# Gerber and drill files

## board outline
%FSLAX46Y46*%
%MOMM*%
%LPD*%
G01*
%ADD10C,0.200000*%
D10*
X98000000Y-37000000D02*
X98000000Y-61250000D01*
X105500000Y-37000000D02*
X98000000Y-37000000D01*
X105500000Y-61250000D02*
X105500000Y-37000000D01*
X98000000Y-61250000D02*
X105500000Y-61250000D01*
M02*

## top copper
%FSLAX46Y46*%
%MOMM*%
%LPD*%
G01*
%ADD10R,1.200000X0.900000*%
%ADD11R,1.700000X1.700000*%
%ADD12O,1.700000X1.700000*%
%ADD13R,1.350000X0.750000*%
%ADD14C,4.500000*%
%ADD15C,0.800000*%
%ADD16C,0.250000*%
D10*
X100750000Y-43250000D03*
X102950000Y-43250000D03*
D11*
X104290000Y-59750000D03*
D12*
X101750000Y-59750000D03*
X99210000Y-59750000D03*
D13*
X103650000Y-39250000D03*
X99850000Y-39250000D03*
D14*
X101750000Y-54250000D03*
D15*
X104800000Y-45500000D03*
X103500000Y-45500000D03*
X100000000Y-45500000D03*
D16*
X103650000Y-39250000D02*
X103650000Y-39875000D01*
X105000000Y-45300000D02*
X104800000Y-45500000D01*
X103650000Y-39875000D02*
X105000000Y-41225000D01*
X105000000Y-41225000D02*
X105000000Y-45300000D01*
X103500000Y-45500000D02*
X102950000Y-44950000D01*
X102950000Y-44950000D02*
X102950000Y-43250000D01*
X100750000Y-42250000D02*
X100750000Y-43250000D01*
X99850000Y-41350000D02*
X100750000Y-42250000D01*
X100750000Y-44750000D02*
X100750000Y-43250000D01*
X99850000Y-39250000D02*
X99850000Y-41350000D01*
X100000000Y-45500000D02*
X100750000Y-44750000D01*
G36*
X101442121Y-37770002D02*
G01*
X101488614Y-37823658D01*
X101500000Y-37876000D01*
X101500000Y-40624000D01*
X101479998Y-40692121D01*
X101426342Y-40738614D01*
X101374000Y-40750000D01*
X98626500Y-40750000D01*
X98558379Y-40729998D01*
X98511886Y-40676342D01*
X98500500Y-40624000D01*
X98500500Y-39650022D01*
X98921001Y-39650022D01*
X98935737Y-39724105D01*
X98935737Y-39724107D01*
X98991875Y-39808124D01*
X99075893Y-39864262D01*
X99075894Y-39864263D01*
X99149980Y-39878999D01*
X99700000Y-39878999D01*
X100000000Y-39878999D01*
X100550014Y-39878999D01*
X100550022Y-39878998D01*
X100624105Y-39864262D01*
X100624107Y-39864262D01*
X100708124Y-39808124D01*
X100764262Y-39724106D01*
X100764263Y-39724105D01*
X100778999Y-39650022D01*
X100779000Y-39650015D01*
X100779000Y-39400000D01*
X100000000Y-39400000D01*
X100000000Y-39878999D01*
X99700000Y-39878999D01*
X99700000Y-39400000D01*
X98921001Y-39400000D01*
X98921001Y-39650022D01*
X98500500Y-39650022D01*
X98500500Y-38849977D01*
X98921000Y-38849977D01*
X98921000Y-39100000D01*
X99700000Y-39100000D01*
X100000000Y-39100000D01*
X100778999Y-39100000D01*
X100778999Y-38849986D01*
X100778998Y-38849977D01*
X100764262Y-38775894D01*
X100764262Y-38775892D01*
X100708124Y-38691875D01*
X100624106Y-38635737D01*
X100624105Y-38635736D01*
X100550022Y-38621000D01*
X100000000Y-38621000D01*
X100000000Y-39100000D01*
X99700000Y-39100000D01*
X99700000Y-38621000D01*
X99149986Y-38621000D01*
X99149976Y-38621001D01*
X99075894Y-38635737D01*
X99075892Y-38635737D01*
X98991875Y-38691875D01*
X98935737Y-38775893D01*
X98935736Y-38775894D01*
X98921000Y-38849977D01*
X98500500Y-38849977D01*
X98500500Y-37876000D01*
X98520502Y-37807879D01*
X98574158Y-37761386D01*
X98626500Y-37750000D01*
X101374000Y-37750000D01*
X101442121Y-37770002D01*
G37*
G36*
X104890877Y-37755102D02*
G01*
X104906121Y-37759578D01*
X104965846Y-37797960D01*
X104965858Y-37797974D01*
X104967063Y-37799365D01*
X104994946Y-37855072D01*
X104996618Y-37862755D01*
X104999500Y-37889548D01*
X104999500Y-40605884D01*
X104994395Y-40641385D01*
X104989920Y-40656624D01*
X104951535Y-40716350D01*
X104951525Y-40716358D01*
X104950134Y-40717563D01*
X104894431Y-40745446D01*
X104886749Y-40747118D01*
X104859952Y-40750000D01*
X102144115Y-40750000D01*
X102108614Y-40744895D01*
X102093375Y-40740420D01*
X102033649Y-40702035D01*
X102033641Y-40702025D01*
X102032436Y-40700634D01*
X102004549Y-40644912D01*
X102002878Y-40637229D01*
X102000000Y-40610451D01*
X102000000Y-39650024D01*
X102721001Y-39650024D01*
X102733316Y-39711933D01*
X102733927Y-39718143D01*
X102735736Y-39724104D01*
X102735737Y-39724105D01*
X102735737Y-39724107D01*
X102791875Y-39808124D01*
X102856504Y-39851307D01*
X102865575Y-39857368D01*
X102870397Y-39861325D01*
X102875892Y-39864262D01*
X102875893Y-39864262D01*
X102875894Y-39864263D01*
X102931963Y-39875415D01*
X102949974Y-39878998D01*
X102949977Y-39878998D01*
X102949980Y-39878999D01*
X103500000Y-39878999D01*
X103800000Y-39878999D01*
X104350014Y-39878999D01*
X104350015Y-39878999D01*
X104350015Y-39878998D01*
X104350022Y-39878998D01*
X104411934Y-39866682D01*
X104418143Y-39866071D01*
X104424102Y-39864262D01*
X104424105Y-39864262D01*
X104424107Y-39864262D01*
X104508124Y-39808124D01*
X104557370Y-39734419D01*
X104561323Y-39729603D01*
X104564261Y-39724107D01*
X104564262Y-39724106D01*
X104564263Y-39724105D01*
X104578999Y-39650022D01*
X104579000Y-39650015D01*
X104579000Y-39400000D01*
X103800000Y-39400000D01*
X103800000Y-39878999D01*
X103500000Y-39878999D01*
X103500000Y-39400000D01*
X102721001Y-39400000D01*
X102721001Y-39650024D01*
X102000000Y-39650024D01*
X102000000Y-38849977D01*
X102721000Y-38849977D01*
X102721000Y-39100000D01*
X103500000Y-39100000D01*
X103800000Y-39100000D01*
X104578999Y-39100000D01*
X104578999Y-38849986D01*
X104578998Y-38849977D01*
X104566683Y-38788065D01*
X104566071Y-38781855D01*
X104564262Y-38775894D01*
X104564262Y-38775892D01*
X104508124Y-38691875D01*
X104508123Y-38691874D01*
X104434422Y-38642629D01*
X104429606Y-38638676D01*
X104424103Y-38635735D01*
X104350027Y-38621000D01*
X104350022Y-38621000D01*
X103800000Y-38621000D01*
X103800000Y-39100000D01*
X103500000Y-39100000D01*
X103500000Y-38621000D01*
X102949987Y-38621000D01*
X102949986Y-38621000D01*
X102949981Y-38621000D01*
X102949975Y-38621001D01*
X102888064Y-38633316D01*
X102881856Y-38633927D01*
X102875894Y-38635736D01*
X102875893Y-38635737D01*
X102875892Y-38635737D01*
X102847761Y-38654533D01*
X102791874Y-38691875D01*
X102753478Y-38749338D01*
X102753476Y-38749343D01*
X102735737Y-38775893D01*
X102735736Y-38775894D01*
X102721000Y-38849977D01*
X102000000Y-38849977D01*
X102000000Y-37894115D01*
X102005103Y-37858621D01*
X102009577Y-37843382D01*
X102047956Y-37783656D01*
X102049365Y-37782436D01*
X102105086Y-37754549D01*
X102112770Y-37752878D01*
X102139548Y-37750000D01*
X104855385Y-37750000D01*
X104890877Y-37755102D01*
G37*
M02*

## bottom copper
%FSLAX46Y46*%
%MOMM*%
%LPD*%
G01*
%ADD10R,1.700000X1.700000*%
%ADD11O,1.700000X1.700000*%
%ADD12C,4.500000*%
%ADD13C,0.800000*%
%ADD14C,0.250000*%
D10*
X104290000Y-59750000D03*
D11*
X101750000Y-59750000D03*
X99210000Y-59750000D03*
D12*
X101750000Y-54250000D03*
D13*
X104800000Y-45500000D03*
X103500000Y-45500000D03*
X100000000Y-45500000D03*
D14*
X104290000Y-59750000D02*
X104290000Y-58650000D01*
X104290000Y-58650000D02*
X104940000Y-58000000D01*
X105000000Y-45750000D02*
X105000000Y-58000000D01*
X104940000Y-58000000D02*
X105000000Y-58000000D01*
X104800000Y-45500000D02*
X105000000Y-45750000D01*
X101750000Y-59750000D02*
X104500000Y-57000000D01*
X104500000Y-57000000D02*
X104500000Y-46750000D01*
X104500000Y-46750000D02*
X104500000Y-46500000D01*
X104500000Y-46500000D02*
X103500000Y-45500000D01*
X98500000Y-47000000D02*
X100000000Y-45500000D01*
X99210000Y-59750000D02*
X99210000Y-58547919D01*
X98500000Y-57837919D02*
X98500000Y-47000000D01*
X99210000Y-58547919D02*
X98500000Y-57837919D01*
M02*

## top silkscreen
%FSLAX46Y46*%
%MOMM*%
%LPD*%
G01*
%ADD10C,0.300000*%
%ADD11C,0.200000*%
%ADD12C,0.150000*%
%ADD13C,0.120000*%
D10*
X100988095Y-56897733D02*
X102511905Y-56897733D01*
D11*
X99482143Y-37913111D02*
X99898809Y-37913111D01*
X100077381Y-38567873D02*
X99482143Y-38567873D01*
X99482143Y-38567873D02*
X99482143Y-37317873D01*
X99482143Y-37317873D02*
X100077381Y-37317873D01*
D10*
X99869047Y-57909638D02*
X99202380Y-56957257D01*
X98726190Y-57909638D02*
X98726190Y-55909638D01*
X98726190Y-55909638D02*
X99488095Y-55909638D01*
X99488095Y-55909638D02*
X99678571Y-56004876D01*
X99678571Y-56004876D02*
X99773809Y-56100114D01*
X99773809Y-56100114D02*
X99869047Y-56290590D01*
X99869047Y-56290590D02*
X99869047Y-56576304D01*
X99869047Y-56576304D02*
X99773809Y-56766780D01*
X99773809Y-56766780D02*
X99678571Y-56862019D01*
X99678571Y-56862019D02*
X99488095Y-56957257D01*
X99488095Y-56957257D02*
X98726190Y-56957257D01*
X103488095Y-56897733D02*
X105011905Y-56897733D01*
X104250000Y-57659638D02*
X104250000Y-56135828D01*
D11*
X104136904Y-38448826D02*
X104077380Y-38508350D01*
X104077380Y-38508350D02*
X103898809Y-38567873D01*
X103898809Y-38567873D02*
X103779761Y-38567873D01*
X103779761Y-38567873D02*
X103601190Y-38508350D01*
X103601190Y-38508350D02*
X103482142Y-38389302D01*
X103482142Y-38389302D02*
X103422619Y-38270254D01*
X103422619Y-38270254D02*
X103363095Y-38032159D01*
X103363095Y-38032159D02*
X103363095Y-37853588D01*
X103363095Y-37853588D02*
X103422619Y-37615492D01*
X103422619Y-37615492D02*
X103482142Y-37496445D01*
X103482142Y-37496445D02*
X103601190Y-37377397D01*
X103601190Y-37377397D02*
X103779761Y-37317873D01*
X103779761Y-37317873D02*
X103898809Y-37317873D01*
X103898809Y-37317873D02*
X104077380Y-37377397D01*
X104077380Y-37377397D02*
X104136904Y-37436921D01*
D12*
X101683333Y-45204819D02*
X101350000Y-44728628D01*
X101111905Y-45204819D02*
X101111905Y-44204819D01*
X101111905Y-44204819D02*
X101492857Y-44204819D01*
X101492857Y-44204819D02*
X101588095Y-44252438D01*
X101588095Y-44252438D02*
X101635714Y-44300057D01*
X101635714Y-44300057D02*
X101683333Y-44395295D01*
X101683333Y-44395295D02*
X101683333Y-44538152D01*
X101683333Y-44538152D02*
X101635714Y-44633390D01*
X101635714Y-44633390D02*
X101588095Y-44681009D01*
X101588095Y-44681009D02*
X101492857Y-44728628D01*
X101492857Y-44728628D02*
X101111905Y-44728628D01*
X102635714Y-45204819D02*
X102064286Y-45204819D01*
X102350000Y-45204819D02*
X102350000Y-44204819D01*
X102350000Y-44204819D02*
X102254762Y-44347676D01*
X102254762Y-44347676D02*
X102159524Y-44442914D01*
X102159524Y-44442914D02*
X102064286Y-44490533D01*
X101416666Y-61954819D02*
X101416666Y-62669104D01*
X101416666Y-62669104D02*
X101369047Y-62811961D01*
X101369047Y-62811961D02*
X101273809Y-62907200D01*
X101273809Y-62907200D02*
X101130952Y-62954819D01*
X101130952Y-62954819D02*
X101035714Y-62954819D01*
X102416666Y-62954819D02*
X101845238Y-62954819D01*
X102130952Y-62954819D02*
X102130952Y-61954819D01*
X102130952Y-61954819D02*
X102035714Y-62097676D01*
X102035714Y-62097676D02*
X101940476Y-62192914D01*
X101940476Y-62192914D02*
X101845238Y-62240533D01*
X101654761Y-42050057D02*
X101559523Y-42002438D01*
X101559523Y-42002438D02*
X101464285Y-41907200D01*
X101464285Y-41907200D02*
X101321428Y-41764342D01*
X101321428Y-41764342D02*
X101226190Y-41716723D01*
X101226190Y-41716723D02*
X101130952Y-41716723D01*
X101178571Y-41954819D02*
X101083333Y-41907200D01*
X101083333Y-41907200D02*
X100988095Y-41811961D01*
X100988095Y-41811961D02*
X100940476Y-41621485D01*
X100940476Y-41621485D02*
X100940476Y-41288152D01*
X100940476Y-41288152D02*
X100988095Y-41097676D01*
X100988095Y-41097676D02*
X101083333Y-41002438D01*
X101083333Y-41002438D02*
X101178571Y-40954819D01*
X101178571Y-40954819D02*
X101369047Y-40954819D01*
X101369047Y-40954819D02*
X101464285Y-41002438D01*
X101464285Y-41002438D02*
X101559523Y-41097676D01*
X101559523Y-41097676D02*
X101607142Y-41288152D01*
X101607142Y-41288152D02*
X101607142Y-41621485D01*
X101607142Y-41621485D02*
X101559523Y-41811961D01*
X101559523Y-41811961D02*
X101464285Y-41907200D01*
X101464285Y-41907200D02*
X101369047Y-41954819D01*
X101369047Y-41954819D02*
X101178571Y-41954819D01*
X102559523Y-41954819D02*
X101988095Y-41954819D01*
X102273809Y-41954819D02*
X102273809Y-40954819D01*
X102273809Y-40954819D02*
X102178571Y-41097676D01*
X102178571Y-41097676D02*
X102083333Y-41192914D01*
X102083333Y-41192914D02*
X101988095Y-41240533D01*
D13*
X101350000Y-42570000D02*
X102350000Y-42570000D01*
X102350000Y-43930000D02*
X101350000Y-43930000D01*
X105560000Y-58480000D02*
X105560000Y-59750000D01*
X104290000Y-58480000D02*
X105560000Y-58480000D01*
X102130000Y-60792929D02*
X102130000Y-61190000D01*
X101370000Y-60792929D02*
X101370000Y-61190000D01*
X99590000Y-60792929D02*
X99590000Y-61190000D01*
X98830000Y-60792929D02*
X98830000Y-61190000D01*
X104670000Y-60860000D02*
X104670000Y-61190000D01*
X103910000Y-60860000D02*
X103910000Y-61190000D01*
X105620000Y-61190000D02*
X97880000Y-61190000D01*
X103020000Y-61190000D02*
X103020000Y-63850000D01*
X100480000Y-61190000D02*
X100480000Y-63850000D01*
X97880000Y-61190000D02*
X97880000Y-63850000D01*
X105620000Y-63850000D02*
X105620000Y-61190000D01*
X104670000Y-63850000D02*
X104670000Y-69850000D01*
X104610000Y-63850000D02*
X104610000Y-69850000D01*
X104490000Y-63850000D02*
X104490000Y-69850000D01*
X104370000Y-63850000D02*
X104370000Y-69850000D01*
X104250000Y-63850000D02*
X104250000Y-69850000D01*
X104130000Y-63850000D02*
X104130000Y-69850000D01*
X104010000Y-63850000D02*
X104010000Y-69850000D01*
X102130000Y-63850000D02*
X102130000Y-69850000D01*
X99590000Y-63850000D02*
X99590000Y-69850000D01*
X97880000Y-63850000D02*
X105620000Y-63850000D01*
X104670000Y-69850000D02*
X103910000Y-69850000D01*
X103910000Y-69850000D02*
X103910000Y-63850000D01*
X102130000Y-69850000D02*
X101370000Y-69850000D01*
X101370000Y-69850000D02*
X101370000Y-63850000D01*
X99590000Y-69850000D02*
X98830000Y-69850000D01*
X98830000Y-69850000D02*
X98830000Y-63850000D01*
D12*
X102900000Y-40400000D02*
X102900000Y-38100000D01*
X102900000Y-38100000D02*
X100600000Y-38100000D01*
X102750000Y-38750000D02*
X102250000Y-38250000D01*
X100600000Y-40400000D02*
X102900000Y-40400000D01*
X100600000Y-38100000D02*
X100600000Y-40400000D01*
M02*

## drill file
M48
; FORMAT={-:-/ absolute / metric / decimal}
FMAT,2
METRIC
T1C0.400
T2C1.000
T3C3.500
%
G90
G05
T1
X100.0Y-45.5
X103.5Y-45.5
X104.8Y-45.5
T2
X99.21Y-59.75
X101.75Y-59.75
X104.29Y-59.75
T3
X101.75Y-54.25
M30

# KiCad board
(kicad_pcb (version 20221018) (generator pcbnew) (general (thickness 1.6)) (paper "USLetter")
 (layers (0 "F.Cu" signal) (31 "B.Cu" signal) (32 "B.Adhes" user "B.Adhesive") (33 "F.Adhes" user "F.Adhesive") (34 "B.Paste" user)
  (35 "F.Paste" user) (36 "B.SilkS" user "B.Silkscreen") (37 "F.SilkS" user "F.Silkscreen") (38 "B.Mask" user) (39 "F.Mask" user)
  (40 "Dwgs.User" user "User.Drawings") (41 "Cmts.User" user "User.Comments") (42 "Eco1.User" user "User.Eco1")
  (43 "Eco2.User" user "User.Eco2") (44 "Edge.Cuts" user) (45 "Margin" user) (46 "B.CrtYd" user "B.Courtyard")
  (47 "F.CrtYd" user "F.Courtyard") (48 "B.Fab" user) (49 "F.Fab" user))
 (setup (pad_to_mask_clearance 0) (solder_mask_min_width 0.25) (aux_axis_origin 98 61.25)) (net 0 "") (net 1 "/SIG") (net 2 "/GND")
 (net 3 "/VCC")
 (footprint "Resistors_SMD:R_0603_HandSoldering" (layer "F.Cu") (at 101.85 43.25)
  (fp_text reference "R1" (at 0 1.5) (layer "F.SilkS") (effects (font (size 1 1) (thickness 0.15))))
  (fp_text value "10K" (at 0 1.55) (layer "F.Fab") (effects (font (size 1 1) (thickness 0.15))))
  (fp_line (start -0.5 -0.68) (end 0.5 -0.68) (stroke (width 0.12) (type solid)) (layer "F.SilkS"))
  (fp_line (start 0.5 0.68) (end -0.5 0.68) (stroke (width 0.12) (type solid)) (layer "F.SilkS"))
  (pad "1" smd rect (at -1.1 0) (size 1.2 0.9) (layers "F.Cu" "F.Paste" "F.Mask") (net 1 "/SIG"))
  (pad "2" smd rect (at 1.1 0) (size 1.2 0.9) (layers "F.Cu" "F.Paste" "F.Mask") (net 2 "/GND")))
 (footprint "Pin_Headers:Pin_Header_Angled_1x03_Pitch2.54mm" (layer "F.Cu") (at 104.29 59.75 -90)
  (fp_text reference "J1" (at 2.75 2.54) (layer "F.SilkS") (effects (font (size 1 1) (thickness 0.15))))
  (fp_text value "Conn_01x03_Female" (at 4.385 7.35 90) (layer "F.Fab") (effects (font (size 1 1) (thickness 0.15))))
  (fp_line (start -1.27 -1.27) (end 0 -1.27) (stroke (width 0.12) (type solid)) (layer "F.SilkS"))
  (fp_line (start -1.27 0) (end -1.27 -1.27) (stroke (width 0.12) (type solid)) (layer "F.SilkS"))
  (fp_line (start 1.042929 2.16) (end 1.44 2.16) (stroke (width 0.12) (type solid)) (layer "F.SilkS"))
  (fp_line (start 1.042929 2.92) (end 1.44 2.92) (stroke (width 0.12) (type solid)) (layer "F.SilkS"))
  (fp_line (start 1.042929 4.7) (end 1.44 4.7) (stroke (width 0.12) (type solid)) (layer "F.SilkS"))
  (fp_line (start 1.042929 5.46) (end 1.44 5.46) (stroke (width 0.12) (type solid)) (layer "F.SilkS"))
  (fp_line (start 1.11 -0.38) (end 1.44 -0.38) (stroke (width 0.12) (type solid)) (layer "F.SilkS"))
  (fp_line (start 1.11 0.38) (end 1.44 0.38) (stroke (width 0.12) (type solid)) (layer "F.SilkS"))
  (fp_line (start 1.44 -1.33) (end 1.44 6.41) (stroke (width 0.12) (type solid)) (layer "F.SilkS"))
  (fp_line (start 1.44 1.27) (end 4.1 1.27) (stroke (width 0.12) (type solid)) (layer "F.SilkS"))
  (fp_line (start 1.44 3.81) (end 4.1 3.81) (stroke (width 0.12) (type solid)) (layer "F.SilkS"))
  (fp_line (start 1.44 6.41) (end 4.1 6.41) (stroke (width 0.12) (type solid)) (layer "F.SilkS"))
  (fp_line (start 4.1 -1.33) (end 1.44 -1.33) (stroke (width 0.12) (type solid)) (layer "F.SilkS"))
  (fp_line (start 4.1 -0.38) (end 10.1 -0.38) (stroke (width 0.12) (type solid)) (layer "F.SilkS"))
  (fp_line (start 4.1 -0.32) (end 10.1 -0.32) (stroke (width 0.12) (type solid)) (layer "F.SilkS"))
  (fp_line (start 4.1 -0.2) (end 10.1 -0.2) (stroke (width 0.12) (type solid)) (layer "F.SilkS"))
  (fp_line (start 4.1 -0.08) (end 10.1 -0.08) (stroke (width 0.12) (type solid)) (layer "F.SilkS"))
  (fp_line (start 4.1 0.04) (end 10.1 0.04) (stroke (width 0.12) (type solid)) (layer "F.SilkS"))
  (fp_line (start 4.1 0.16) (end 10.1 0.16) (stroke (width 0.12) (type solid)) (layer "F.SilkS"))
  (fp_line (start 4.1 0.28) (end 10.1 0.28) (stroke (width 0.12) (type solid)) (layer "F.SilkS"))
  (fp_line (start 4.1 2.16) (end 10.1 2.16) (stroke (width 0.12) (type solid)) (layer "F.SilkS"))
  (fp_line (start 4.1 4.7) (end 10.1 4.7) (stroke (width 0.12) (type solid)) (layer "F.SilkS"))
  (fp_line (start 4.1 6.41) (end 4.1 -1.33) (stroke (width 0.12) (type solid)) (layer "F.SilkS"))
  (fp_line (start 10.1 -0.38) (end 10.1 0.38) (stroke (width 0.12) (type solid)) (layer "F.SilkS"))
  (fp_line (start 10.1 0.38) (end 4.1 0.38) (stroke (width 0.12) (type solid)) (layer "F.SilkS"))
  (fp_line (start 10.1 2.16) (end 10.1 2.92) (stroke (width 0.12) (type solid)) (layer "F.SilkS"))
  (fp_line (start 10.1 2.92) (end 4.1 2.92) (stroke (width 0.12) (type solid)) (layer "F.SilkS"))
  (fp_line (start 10.1 4.7) (end 10.1 5.46) (stroke (width 0.12) (type solid)) (layer "F.SilkS"))
  (fp_line (start 10.1 5.46) (end 4.1 5.46) (stroke (width 0.12) (type solid)) (layer "F.SilkS"))
  (pad "1" thru_hole rect (at 0 0 270) (size 1.7 1.7) (drill 1) (layers "*.Cu" "*.Mask") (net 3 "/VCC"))
  (pad "2" thru_hole oval (at 0 2.54 270) (size 1.7 1.7) (drill 1) (layers "*.Cu" "*.Mask") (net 2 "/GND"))
  (pad "3" thru_hole oval (at 0 5.08 270) (size 1.7 1.7) (drill 1) (layers "*.Cu" "*.Mask") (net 1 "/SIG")))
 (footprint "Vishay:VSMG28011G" (layer "F.Cu") (at 101.75 39.25 180)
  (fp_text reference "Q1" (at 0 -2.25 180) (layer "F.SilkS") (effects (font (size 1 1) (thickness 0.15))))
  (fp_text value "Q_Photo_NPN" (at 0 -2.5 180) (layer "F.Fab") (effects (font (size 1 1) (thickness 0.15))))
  (fp_line (start -1.15 -1.15) (end -1.15 1.15) (stroke (width 0.15) (type solid)) (layer "F.SilkS"))
  (fp_line (start -1.15 1.15) (end 1.15 1.15) (stroke (width 0.15) (type solid)) (layer "F.SilkS"))
  (fp_line (start -1 0.5) (end -0.5 1) (stroke (width 0.15) (type solid)) (layer "F.SilkS"))
  (fp_line (start 1.15 -1.15) (end -1.15 -1.15) (stroke (width 0.15) (type solid)) (layer "F.SilkS"))
  (fp_line (start 1.15 1.15) (end 1.15 -1.15) (stroke (width 0.15) (type solid)) (layer "F.SilkS"))
  (pad "1" smd rect (at -1.9 0 180) (size 1.35 0.75) (layers "F.Cu" "F.Paste" "F.Mask") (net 3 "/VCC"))
  (pad "2" smd rect (at 1.9 0 180) (size 1.35 0.75) (layers "F.Cu" "F.Paste" "F.Mask") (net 1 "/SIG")))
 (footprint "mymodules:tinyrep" (layer "B.Cu") (at 101.75 44.5 90)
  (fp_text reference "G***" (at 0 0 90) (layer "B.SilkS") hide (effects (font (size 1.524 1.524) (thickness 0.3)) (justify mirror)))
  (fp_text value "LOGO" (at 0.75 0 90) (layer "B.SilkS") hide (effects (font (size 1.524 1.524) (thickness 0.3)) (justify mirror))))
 (gr_line (start 98 37) (end 98 61.25) (stroke (width 0.2) (type solid)) (layer "Edge.Cuts"))
 (gr_line (start 105.5 37) (end 98 37) (stroke (width 0.2) (type solid)) (layer "Edge.Cuts"))
 (gr_line (start 105.5 61.25) (end 105.5 37) (stroke (width 0.2) (type solid)) (layer "Edge.Cuts"))
 (gr_line (start 98 61.25) (end 105.5 61.25) (stroke (width 0.2) (type solid)) (layer "Edge.Cuts"))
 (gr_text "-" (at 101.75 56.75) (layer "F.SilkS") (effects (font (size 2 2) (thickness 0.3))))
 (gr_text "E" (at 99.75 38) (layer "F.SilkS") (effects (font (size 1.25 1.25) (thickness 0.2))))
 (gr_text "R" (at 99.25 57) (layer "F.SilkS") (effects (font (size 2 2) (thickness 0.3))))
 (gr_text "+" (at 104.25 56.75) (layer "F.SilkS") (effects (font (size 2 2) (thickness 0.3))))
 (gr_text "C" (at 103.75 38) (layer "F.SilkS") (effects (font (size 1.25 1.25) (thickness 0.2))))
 (via (at 101.75 54.25) (size 4.5) (drill 3.5) (layers "F.Cu" "B.Cu") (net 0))
 (segment (start 103.65 39.25) (end 103.65 39.875) (width 0.25) (layer "F.Cu") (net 3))
 (segment (start 105 45.3) (end 104.8 45.5) (width 0.25) (layer "F.Cu") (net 3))
 (segment (start 103.65 39.875) (end 105 41.225) (width 0.25) (layer "F.Cu") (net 3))
 (segment (start 105 41.225) (end 105 45.3) (width 0.25) (layer "F.Cu") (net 3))
 (via (at 104.8 45.5) (size 0.8) (drill 0.4) (layers "F.Cu" "B.Cu") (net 3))
 (segment (start 104.29 59.75) (end 104.29 58.65) (width 0.25) (layer "B.Cu") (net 3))
 (segment (start 104.29 58.65) (end 104.94 58) (width 0.25) (layer "B.Cu") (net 3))
 (segment (start 105 45.75) (end 105 58) (width 0.25) (layer "B.Cu") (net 3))
 (segment (start 104.94 58) (end 105 58) (width 0.25) (layer "B.Cu") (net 3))
 (segment (start 104.8 45.5) (end 105 45.75) (width 0.25) (layer "B.Cu") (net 3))
 (segment (start 103.5 45.5) (end 102.95 44.95) (width 0.25) (layer "F.Cu") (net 2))
 (segment (start 102.95 44.95) (end 102.95 43.25) (width 0.25) (layer "F.Cu") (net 2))
 (via (at 103.5 45.5) (size 0.8) (drill 0.4) (layers "F.Cu" "B.Cu") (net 2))
 (segment (start 101.75 59.75) (end 104.5 57) (width 0.25) (layer "B.Cu") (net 2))
 (segment (start 104.5 57) (end 104.5 46.75) (width 0.25) (layer "B.Cu") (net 2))
 (segment (start 104.5 46.75) (end 104.5 46.5) (width 0.25) (layer "B.Cu") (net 2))
 (segment (start 104.5 46.5) (end 103.5 45.5) (width 0.25) (layer "B.Cu") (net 2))
 (segment (start 100.75 42.25) (end 100.75 43.25) (width 0.25) (layer "F.Cu") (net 1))
 (segment (start 99.85 41.35) (end 100.75 42.25) (width 0.25) (layer "F.Cu") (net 1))
 (segment (start 100.75 44.75) (end 100.75 43.25) (width 0.25) (layer "F.Cu") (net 1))
 (segment (start 99.85 39.25) (end 99.85 41.35) (width 0.25) (layer "F.Cu") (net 1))
 (segment (start 100 45.5) (end 100.75 44.75) (width 0.25) (layer "F.Cu") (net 1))
 (via (at 100 45.5) (size 0.8) (drill 0.4) (layers "F.Cu" "B.Cu") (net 1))
 (segment (start 98.5 47) (end 100 45.5) (width 0.25) (layer "B.Cu") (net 1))
 (segment (start 99.21 59.75) (end 99.21 58.547919) (width 0.25) (layer "B.Cu") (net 1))
 (segment (start 98.5 57.837919) (end 98.5 47) (width 0.25) (layer "B.Cu") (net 1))
 (segment (start 99.21 58.547919) (end 98.5 57.837919) (width 0.25) (layer "B.Cu") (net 1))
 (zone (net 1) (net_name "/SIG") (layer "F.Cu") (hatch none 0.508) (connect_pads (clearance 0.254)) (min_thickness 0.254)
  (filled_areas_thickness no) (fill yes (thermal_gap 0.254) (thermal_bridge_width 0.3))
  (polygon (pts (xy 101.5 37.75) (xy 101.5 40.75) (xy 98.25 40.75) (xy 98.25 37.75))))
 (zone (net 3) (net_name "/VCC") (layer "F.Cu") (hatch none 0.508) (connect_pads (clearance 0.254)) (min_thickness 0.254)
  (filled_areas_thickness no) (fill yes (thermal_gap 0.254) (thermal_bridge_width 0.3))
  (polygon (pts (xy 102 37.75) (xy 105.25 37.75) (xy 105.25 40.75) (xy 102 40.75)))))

